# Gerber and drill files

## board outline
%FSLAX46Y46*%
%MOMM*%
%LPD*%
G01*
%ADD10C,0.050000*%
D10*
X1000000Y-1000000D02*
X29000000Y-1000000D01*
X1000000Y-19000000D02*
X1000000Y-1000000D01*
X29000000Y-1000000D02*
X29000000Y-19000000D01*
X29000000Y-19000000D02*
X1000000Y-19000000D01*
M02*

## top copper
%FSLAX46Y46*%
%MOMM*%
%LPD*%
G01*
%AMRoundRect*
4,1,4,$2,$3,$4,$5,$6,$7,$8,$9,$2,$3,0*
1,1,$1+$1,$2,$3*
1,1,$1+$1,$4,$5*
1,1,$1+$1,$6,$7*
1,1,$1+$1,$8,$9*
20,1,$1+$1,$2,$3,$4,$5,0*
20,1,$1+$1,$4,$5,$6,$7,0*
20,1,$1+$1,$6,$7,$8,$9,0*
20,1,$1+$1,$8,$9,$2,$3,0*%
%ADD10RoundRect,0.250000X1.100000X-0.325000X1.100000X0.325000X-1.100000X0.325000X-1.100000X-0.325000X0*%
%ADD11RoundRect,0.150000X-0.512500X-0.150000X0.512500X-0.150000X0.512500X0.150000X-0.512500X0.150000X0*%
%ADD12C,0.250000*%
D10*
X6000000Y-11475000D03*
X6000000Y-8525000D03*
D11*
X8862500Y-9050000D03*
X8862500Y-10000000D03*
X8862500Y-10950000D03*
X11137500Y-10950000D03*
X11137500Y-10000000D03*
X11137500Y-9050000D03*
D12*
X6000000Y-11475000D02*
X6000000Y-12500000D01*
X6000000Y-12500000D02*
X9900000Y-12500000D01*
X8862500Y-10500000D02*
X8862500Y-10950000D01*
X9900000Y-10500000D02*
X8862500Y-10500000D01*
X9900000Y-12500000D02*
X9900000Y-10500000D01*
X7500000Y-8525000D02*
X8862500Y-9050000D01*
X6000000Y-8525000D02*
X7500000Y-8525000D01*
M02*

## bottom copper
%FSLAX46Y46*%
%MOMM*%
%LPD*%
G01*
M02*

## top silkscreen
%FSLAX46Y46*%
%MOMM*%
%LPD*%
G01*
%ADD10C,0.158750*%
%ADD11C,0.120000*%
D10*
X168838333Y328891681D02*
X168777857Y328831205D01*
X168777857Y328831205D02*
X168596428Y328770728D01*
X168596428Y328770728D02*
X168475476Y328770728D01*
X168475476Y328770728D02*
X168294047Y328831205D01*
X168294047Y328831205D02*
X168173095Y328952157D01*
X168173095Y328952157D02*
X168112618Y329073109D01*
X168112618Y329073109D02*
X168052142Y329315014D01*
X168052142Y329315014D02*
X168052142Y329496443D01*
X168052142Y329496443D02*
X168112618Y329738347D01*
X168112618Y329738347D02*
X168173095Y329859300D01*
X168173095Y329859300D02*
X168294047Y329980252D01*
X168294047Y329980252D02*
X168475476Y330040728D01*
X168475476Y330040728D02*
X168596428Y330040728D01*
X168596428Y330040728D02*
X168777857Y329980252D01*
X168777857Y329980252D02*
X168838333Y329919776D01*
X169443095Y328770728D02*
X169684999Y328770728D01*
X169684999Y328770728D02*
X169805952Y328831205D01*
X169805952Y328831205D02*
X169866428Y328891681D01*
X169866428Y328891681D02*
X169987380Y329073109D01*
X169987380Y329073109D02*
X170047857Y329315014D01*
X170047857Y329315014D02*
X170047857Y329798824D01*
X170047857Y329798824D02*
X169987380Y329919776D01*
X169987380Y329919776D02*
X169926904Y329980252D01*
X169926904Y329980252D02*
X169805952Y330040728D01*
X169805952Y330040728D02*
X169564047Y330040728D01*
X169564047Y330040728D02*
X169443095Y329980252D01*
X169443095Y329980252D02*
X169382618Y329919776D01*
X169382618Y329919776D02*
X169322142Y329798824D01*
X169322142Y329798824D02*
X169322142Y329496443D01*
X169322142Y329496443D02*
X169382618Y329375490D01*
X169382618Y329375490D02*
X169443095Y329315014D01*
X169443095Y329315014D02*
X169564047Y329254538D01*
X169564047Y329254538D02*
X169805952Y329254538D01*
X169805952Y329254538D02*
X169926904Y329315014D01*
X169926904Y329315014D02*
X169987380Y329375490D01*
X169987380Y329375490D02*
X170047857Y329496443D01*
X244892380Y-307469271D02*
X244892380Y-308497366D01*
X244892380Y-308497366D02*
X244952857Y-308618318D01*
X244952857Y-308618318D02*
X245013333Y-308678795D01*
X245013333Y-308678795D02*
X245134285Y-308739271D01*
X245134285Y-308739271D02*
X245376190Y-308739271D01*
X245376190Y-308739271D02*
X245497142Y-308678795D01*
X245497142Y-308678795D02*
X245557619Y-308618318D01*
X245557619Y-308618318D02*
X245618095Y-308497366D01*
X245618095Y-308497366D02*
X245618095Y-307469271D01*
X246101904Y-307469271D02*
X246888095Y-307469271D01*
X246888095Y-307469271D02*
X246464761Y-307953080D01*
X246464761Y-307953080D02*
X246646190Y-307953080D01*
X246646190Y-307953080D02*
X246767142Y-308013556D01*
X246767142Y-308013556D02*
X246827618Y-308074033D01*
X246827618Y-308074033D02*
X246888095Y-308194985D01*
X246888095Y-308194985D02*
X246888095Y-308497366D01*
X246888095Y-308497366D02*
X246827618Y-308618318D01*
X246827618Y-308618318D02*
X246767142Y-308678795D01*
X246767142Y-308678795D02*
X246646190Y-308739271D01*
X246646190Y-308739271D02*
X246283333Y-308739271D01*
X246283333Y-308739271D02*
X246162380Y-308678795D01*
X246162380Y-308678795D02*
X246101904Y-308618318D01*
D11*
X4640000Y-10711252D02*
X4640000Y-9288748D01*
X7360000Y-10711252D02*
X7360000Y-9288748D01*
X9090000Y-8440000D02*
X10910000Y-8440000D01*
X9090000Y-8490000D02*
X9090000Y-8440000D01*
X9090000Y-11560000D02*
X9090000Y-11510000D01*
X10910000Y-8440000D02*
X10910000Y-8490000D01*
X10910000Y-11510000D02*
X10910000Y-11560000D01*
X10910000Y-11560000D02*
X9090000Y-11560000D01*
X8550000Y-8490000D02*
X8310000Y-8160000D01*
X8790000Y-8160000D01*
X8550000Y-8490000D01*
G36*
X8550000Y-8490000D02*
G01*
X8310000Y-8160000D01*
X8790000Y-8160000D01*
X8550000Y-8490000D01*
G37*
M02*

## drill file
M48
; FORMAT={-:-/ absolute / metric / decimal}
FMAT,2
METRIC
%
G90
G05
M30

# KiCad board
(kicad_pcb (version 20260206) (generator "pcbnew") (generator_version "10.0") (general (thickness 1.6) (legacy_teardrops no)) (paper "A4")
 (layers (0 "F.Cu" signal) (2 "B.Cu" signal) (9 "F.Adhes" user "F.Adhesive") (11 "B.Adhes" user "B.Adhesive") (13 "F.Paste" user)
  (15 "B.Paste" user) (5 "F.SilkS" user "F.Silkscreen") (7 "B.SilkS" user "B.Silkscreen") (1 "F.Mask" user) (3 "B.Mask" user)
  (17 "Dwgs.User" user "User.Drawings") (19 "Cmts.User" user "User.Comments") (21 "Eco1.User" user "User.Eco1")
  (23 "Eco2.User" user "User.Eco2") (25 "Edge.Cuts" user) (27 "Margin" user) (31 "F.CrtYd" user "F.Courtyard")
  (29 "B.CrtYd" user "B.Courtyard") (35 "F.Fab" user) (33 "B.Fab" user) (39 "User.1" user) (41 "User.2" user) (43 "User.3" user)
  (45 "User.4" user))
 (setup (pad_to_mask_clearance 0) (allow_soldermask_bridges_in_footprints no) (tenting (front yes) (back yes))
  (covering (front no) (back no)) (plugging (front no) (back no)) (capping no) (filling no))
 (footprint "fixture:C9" (layer "F.Cu") (at 6 10 90)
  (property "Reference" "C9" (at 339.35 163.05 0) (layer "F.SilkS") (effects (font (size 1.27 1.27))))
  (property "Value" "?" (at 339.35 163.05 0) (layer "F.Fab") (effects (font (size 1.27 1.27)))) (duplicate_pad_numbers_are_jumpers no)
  (fp_line (start -0.711252 -1.36) (end 0.711252 -1.36) (stroke (width 0.12) (type solid)) (layer "F.SilkS"))
  (fp_line (start -0.711252 1.36) (end 0.711252 1.36) (stroke (width 0.12) (type solid)) (layer "F.SilkS"))
  (pad "1" smd roundrect (at -1.475 0 90) (size 1.15 2.7) (layers "F.Cu" "F.Mask" "F.Paste") (roundrect_rratio 0.217391) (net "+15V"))
  (pad "2" smd roundrect (at 1.475 0 90) (size 1.15 2.7) (layers "F.Cu" "F.Mask" "F.Paste") (roundrect_rratio 0.217391) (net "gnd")))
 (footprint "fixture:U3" (layer "F.Cu") (at 10 10)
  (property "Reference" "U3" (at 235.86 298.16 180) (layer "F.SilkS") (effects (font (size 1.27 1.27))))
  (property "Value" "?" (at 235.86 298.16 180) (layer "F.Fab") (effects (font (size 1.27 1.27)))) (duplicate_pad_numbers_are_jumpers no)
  (fp_line (start -0.91 -1.56) (end 0.91 -1.56) (stroke (width 0.12) (type solid)) (layer "F.SilkS"))
  (fp_line (start -0.91 -1.51) (end -0.91 -1.56) (stroke (width 0.12) (type solid)) (layer "F.SilkS"))
  (fp_line (start -0.91 1.56) (end -0.91 1.51) (stroke (width 0.12) (type solid)) (layer "F.SilkS"))
  (fp_line (start 0.91 -1.56) (end 0.91 -1.51) (stroke (width 0.12) (type solid)) (layer "F.SilkS"))
  (fp_line (start 0.91 1.51) (end 0.91 1.56) (stroke (width 0.12) (type solid)) (layer "F.SilkS"))
  (fp_line (start 0.91 1.56) (end -0.91 1.56) (stroke (width 0.12) (type solid)) (layer "F.SilkS"))
  (fp_poly (pts (xy -1.45 -1.51) (xy -1.69 -1.84) (xy -1.21 -1.84)) (stroke (width 0.12) (type solid)) (fill yes) (layer "F.SilkS"))
  (pad "1" smd roundrect (at -1.1375 -0.95) (size 1.325 0.6) (layers "F.Cu" "F.Mask" "F.Paste") (roundrect_rratio 0.25) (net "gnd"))
  (pad "2" smd roundrect (at -1.1375 0) (size 1.325 0.6) (layers "F.Cu" "F.Mask" "F.Paste") (roundrect_rratio 0.25) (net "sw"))
  (pad "3" smd roundrect (at -1.1375 0.95) (size 1.325 0.6) (layers "F.Cu" "F.Mask" "F.Paste") (roundrect_rratio 0.25) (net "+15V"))
  (pad "4" smd roundrect (at 1.1375 0.95) (size 1.325 0.6) (layers "F.Cu" "F.Mask" "F.Paste") (roundrect_rratio 0.25) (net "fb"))
  (pad "5" smd roundrect (at 1.1375 0) (size 1.325 0.6) (layers "F.Cu" "F.Mask" "F.Paste") (roundrect_rratio 0.25) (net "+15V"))
  (pad "6" smd roundrect (at 1.1375 -0.95) (size 1.325 0.6) (layers "F.Cu" "F.Mask" "F.Paste") (roundrect_rratio 0.25) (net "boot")))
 (gr_line (start 1 1) (end 29 1) (stroke (width 0.05) (type default)) (layer "Edge.Cuts"))
 (gr_line (start 1 19) (end 1 1) (stroke (width 0.05) (type default)) (layer "Edge.Cuts"))
 (gr_line (start 29 1) (end 29 19) (stroke (width 0.05) (type default)) (layer "Edge.Cuts"))
 (gr_line (start 29 19) (end 1 19) (stroke (width 0.05) (type default)) (layer "Edge.Cuts"))
 (segment (start 6 11.475) (end 6 12.5) (width 0.25) (layer "F.Cu") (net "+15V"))
 (segment (start 6 12.5) (end 9.9 12.5) (width 0.25) (layer "F.Cu") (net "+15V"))
 (segment (start 8.8625 10.5) (end 8.8625 10.95) (width 0.25) (layer "F.Cu") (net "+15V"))
 (segment (start 9.9 10.5) (end 8.8625 10.5) (width 0.25) (layer "F.Cu") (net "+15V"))
 (segment (start 9.9 12.5) (end 9.9 10.5) (width 0.25) (layer "F.Cu") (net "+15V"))
 (segment (start 7.5 8.525) (end 8.8625 9.05) (width 0.25) (layer "F.Cu") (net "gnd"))
 (segment (start 6 8.525) (end 7.5 8.525) (width 0.25) (layer "F.Cu") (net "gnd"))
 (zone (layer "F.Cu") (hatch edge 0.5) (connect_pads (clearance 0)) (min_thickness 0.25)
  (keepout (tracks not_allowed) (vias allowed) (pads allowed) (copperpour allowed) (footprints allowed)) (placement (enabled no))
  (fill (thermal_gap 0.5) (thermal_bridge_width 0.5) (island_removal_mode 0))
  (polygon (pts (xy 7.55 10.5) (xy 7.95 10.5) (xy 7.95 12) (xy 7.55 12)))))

